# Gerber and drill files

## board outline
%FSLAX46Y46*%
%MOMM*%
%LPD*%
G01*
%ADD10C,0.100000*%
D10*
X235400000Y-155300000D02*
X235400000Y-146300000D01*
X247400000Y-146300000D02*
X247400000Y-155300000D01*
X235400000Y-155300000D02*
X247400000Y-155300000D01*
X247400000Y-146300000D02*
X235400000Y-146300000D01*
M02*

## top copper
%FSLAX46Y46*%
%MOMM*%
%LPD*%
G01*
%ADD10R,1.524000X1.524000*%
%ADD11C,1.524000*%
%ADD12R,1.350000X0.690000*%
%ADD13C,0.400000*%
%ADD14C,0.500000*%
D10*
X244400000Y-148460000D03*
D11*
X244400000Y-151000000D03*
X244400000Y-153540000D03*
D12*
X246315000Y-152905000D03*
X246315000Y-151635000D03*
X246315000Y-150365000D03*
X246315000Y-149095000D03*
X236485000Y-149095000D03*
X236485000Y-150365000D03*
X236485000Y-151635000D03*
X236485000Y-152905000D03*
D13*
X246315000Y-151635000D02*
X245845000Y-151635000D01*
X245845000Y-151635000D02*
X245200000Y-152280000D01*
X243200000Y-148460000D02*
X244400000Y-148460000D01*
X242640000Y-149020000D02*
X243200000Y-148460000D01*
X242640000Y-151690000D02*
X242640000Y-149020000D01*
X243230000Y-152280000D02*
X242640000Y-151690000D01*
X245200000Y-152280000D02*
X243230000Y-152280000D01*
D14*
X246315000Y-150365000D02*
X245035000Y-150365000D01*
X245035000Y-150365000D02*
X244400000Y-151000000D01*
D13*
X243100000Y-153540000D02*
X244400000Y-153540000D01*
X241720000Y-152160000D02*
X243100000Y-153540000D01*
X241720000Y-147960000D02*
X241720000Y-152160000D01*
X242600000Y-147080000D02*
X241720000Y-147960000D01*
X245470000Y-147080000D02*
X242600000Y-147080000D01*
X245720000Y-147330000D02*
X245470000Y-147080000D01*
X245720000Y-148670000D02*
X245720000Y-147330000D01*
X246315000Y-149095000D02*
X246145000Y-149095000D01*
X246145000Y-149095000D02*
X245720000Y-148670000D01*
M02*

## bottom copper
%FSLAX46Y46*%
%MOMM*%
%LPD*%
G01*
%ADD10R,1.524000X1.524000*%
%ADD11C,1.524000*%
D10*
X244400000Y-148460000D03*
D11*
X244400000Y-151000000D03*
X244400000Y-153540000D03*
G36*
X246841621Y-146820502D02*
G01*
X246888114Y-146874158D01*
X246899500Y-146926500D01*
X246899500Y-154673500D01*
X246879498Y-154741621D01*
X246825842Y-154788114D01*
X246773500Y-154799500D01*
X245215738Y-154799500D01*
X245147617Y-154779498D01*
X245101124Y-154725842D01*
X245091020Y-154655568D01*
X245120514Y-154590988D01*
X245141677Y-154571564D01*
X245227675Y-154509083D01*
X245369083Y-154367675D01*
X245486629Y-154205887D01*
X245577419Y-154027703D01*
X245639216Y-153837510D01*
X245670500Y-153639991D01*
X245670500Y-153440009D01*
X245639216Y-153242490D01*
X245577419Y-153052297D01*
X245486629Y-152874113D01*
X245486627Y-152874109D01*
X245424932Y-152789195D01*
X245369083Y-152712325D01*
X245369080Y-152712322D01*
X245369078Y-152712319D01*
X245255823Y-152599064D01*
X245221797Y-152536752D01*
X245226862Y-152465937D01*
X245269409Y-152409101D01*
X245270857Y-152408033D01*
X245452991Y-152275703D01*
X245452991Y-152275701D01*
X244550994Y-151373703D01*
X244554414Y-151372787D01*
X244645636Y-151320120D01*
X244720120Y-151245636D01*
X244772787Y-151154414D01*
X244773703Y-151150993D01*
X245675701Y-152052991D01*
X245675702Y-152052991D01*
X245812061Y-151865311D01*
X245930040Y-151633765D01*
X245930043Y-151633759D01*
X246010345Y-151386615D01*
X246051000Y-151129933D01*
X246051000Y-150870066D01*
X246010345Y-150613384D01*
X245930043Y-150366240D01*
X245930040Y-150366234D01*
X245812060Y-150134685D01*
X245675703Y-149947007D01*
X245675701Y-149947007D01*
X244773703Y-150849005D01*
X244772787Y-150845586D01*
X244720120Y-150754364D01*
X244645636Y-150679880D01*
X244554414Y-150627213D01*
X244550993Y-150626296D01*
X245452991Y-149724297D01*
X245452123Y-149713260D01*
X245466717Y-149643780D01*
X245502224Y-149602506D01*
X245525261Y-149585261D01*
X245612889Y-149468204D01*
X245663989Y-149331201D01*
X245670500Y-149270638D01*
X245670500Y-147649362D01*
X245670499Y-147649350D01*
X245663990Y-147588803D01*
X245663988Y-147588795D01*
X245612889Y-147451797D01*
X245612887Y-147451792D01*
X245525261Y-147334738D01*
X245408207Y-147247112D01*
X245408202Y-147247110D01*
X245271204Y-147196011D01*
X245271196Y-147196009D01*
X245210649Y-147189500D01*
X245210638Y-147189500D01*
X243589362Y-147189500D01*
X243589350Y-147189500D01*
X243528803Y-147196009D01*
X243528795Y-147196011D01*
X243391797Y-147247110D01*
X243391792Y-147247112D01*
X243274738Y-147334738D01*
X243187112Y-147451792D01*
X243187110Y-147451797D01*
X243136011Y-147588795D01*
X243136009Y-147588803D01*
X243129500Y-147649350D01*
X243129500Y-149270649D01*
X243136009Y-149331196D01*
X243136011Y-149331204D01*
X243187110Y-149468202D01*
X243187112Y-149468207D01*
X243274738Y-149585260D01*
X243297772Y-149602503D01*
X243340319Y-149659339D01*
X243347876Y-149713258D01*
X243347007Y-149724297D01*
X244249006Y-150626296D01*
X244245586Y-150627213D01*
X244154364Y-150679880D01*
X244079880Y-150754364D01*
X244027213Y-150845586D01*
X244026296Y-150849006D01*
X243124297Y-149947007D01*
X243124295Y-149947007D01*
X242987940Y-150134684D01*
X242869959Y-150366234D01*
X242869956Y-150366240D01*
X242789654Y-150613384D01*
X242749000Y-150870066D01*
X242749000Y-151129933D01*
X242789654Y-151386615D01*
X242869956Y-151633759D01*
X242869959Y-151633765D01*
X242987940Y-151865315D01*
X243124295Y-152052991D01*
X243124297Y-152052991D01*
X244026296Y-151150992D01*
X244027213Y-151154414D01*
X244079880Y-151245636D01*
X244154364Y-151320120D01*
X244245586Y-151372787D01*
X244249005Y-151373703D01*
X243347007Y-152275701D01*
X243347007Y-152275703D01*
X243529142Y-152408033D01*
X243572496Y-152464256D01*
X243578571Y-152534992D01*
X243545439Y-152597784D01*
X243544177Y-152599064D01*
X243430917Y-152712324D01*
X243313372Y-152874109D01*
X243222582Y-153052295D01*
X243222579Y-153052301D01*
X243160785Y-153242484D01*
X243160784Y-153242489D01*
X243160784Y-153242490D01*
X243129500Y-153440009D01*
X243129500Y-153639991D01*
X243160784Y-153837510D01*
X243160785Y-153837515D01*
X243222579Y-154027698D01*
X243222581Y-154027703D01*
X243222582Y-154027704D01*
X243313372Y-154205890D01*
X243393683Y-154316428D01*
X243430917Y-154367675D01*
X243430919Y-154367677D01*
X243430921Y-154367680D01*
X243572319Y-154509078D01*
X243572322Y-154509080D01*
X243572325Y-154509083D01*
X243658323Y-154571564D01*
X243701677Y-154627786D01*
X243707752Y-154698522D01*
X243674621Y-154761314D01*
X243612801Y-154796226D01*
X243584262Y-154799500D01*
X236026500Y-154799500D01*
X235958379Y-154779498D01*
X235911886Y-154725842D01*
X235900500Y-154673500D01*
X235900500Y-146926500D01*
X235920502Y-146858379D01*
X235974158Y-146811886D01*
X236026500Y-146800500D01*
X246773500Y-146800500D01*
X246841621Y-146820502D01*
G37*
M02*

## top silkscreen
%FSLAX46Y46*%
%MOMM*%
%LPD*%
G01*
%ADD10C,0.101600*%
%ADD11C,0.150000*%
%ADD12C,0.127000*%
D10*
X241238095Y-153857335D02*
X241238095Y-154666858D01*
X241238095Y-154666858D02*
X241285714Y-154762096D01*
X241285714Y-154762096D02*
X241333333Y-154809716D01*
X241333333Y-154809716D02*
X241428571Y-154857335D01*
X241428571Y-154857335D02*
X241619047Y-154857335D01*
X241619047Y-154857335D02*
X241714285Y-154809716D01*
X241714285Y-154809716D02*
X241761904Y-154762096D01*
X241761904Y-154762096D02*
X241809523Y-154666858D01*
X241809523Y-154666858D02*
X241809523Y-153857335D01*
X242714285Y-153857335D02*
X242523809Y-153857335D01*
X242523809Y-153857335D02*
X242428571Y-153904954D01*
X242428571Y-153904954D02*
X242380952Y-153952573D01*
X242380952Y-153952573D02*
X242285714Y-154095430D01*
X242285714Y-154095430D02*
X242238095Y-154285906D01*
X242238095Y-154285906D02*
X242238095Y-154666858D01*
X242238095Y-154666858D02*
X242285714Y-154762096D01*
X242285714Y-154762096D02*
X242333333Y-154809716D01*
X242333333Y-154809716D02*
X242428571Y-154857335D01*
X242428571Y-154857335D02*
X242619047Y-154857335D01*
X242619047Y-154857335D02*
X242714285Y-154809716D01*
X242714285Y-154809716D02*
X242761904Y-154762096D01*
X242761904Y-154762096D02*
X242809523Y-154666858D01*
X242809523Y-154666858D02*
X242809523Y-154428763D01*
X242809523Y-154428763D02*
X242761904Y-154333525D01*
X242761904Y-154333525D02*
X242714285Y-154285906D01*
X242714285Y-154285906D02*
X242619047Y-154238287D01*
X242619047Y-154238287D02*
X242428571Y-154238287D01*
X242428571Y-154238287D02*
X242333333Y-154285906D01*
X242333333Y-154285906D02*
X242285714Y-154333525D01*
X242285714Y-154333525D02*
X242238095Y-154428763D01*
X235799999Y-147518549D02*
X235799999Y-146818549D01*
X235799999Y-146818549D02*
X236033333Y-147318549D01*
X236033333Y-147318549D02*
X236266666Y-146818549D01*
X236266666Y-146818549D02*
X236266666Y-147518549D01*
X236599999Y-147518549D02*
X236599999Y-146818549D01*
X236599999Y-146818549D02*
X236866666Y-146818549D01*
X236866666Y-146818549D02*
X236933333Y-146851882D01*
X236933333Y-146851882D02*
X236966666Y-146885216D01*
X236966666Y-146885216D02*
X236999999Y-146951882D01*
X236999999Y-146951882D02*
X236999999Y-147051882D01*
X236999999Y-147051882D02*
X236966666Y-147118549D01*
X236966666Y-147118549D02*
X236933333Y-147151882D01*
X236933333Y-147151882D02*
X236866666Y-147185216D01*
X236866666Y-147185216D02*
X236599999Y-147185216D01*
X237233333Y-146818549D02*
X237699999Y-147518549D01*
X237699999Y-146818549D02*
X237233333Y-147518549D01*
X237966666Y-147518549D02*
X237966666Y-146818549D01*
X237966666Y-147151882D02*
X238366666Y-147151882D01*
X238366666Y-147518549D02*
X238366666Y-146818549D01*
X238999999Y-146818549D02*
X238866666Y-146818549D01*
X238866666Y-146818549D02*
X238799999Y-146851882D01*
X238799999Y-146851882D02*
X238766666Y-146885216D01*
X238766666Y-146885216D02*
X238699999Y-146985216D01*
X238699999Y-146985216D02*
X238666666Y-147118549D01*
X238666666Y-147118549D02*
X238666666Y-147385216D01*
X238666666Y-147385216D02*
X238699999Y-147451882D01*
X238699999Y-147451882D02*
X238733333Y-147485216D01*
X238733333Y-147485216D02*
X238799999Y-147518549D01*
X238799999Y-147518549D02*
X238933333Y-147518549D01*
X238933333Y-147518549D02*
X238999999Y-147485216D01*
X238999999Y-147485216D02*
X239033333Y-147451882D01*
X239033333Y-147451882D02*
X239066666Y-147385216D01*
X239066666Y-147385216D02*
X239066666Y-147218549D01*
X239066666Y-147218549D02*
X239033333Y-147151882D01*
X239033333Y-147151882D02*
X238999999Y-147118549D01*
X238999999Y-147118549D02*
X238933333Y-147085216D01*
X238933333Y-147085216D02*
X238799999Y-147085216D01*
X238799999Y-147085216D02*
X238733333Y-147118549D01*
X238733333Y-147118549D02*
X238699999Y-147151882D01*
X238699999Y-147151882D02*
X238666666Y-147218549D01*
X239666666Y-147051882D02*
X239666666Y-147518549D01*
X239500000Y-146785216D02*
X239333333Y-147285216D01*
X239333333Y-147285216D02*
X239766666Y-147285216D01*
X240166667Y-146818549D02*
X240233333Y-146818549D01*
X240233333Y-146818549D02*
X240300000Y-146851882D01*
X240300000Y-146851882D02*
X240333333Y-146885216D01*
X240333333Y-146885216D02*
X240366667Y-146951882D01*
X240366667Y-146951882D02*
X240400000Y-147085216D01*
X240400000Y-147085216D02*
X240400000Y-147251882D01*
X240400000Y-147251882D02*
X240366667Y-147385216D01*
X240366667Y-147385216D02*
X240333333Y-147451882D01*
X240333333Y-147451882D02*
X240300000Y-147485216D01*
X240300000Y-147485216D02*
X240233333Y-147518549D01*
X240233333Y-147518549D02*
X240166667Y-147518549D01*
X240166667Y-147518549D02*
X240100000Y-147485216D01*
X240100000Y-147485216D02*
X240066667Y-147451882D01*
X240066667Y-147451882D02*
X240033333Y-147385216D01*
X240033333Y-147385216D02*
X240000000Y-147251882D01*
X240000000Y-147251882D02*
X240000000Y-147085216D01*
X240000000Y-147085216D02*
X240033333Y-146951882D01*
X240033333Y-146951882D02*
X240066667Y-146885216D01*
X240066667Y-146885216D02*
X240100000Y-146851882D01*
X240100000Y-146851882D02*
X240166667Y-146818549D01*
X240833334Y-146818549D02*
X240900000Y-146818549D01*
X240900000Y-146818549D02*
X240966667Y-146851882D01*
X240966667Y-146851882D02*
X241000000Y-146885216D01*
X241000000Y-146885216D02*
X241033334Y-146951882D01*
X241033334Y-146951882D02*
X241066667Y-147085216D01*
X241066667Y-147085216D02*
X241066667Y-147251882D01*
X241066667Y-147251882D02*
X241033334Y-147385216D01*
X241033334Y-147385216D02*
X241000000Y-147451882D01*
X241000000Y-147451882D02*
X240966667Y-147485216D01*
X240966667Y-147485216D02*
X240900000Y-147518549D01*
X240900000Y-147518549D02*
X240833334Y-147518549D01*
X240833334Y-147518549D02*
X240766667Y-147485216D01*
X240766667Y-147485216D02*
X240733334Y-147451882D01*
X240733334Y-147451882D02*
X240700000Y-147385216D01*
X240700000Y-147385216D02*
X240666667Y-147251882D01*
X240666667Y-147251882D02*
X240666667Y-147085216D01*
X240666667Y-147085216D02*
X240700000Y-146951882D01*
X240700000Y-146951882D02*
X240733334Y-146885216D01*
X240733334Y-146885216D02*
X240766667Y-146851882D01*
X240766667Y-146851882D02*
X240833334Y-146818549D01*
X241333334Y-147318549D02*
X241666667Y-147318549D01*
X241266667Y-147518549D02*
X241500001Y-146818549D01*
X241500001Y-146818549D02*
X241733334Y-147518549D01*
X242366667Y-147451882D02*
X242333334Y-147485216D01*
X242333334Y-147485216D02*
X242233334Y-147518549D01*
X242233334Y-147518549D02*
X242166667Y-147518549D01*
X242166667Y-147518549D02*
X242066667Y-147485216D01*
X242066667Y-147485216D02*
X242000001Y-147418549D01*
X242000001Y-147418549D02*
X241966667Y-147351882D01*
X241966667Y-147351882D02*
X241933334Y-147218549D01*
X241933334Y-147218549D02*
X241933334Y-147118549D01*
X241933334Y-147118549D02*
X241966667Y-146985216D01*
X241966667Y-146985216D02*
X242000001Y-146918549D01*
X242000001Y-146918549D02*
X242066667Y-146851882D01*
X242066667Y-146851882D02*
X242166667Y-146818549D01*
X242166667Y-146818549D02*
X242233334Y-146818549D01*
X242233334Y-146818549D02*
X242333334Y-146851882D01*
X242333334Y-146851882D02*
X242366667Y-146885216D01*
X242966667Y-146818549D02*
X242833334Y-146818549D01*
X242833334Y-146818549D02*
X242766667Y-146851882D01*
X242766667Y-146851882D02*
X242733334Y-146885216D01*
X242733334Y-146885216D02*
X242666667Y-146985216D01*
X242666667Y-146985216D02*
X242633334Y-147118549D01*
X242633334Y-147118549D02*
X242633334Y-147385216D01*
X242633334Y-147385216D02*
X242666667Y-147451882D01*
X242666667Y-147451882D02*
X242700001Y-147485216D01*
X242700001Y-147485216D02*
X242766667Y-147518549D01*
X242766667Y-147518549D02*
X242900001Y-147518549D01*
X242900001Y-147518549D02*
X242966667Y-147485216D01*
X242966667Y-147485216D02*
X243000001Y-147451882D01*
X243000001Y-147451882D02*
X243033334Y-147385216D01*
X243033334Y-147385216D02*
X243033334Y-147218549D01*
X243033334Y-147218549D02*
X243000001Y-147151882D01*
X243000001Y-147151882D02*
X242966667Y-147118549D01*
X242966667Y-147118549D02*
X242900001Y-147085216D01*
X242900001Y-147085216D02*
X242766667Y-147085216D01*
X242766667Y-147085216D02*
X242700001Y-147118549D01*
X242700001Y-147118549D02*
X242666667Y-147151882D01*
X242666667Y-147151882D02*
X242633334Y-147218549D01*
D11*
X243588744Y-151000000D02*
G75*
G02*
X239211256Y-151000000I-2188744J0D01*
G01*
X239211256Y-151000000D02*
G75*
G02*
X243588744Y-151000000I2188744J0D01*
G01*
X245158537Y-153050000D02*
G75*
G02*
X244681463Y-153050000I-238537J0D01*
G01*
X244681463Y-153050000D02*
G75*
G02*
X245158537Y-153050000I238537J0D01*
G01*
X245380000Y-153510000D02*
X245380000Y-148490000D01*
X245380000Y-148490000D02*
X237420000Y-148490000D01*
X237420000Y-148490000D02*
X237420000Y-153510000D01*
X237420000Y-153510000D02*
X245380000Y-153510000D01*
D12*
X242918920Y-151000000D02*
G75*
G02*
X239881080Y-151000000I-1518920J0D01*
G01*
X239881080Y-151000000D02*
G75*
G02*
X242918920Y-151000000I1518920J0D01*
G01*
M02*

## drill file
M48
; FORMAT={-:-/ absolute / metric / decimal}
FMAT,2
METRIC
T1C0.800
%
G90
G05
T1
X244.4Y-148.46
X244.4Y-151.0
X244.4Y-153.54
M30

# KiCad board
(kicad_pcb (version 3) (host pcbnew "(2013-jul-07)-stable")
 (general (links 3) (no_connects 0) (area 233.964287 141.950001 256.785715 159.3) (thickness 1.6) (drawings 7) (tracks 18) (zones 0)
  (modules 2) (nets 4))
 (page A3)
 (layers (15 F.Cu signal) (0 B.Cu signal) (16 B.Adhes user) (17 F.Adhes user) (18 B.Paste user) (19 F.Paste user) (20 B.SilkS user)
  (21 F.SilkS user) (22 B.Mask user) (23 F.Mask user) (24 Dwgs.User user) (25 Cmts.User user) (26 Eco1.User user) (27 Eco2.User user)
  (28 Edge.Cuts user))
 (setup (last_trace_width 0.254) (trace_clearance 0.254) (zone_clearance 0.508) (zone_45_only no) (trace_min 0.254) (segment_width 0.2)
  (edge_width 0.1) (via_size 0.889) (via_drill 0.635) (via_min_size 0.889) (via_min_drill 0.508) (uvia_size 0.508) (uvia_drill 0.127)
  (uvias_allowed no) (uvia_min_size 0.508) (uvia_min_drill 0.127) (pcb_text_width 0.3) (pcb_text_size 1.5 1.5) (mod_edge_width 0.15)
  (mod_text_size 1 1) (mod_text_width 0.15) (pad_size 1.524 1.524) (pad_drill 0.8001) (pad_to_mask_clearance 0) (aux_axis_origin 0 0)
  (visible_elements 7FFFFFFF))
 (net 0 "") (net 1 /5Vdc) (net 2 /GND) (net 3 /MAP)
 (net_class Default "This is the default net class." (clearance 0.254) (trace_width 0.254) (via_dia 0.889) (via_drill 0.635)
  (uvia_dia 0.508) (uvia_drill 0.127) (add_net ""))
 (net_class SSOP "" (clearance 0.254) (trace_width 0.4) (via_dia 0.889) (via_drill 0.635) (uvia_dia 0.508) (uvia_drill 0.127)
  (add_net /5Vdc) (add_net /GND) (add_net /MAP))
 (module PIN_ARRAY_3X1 (layer B.Cu) (at 244.4 151 270)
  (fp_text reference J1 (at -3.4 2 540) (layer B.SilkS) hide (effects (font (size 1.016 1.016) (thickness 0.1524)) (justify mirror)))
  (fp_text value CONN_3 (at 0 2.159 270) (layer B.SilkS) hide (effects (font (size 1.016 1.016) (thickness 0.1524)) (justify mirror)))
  (pad 1 thru_hole rect (at -2.54 0 270) (size 1.524 1.524) (drill 0.8001) (layers *.Cu *.Mask B.SilkS) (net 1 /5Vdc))
  (pad 2 thru_hole circle (at 0 0 270) (size 1.524 1.524) (drill 0.8001) (layers *.Cu *.Mask B.SilkS) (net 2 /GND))
  (pad 3 thru_hole circle (at 2.54 0 270) (size 1.524 1.524) (drill 0.8001) (layers *.Cu *.Mask B.SilkS) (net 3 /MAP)))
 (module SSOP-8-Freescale (layer F.Cu) (at 241.4 151)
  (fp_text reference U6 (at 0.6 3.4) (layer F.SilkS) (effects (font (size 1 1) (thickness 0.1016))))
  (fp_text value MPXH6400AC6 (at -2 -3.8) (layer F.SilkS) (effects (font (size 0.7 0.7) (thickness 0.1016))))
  (fp_circle (center 0 0) (end 2.15 0.41) (layer F.SilkS) (width 0.15))
  (fp_circle (center 3.52 2.05) (end 3.32 1.92) (layer F.SilkS) (width 0.15))
  (fp_line (start 3.98 2.51) (end 3.98 -2.51) (layer F.SilkS) (width 0.15))
  (fp_line (start 3.98 -2.51) (end -3.98 -2.51) (layer F.SilkS) (width 0.15))
  (fp_line (start -3.98 -2.51) (end -3.98 2.51) (layer F.SilkS) (width 0.15))
  (fp_line (start -3.98 2.51) (end 3.98 2.51) (layer F.SilkS) (width 0.15))
  (fp_circle (center 0 0) (end 1.51892 0) (layer F.SilkS) (width 0.127))
  (pad 1 smd rect (at 4.915 1.905) (size 1.35 0.69) (layers F.Cu F.Paste F.Mask))
  (pad 2 smd rect (at 4.915 0.635) (size 1.35 0.69) (layers F.Cu F.Paste F.Mask) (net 1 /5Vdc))
  (pad 3 smd rect (at 4.915 -0.635) (size 1.35 0.69) (layers F.Cu F.Paste F.Mask) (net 2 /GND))
  (pad 4 smd rect (at 4.915 -1.905) (size 1.35 0.69) (layers F.Cu F.Paste F.Mask) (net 3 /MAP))
  (pad 5 smd rect (at -4.915 -1.905) (size 1.35 0.69) (layers F.Cu F.Paste F.Mask))
  (pad 6 smd rect (at -4.915 -0.635) (size 1.35 0.69) (layers F.Cu F.Paste F.Mask))
  (pad 7 smd rect (at -4.915 0.635) (size 1.35 0.69) (layers F.Cu F.Paste F.Mask))
  (pad 8 smd rect (at -4.915 1.905) (size 1.35 0.69) (layers F.Cu F.Paste F.Mask)))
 (gr_line (start 235.4 155.3) (end 235.4 146.3) (angle 90) (layer Edge.Cuts) (width 0.1))
 (gr_line (start 247.4 146.3) (end 247.4 155.3) (angle 90) (layer Edge.Cuts) (width 0.1))
 (gr_line (start 235.4 155.3) (end 247.4 155.3) (angle 90) (layer Edge.Cuts) (width 0.1))
 (gr_line (start 247.4 146.3) (end 235.4 146.3) (angle 90) (layer Edge.Cuts) (width 0.1))
 (segment (start 246.315 151.635) (end 245.845 151.635) (width 0.4) (layer F.Cu) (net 1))
 (segment (start 245.845 151.635) (end 245.2 152.28) (width 0.4) (layer F.Cu) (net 1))
 (segment (start 243.2 148.46) (end 244.4 148.46) (width 0.4) (layer F.Cu) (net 1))
 (segment (start 242.64 149.02) (end 243.2 148.46) (width 0.4) (layer F.Cu) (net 1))
 (segment (start 242.64 151.69) (end 242.64 149.02) (width 0.4) (layer F.Cu) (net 1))
 (segment (start 243.23 152.28) (end 242.64 151.69) (width 0.4) (layer F.Cu) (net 1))
 (segment (start 245.2 152.28) (end 243.23 152.28) (width 0.4) (layer F.Cu) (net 1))
 (segment (start 246.315 150.365) (end 245.035 150.365) (width 0.5) (layer F.Cu) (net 2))
 (segment (start 245.035 150.365) (end 244.4 151) (width 0.5) (layer F.Cu) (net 2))
 (segment (start 243.1 153.54) (end 244.4 153.54) (width 0.4) (layer F.Cu) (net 3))
 (segment (start 241.72 152.16) (end 243.1 153.54) (width 0.4) (layer F.Cu) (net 3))
 (segment (start 241.72 147.96) (end 241.72 152.16) (width 0.4) (layer F.Cu) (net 3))
 (segment (start 242.6 147.08) (end 241.72 147.96) (width 0.4) (layer F.Cu) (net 3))
 (segment (start 245.47 147.08) (end 242.6 147.08) (width 0.4) (layer F.Cu) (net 3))
 (segment (start 245.72 147.33) (end 245.47 147.08) (width 0.4) (layer F.Cu) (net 3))
 (segment (start 245.72 148.67) (end 245.72 147.33) (width 0.4) (layer F.Cu) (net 3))
 (segment (start 246.315 149.095) (end 246.145 149.095) (width 0.4) (layer F.Cu) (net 3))
 (segment (start 246.145 149.095) (end 245.72 148.67) (width 0.4) (layer F.Cu) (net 3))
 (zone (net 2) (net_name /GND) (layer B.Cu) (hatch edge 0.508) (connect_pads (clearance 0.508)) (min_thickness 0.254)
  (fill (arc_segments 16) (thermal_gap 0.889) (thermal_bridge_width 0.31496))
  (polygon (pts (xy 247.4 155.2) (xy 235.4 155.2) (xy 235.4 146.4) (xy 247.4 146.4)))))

